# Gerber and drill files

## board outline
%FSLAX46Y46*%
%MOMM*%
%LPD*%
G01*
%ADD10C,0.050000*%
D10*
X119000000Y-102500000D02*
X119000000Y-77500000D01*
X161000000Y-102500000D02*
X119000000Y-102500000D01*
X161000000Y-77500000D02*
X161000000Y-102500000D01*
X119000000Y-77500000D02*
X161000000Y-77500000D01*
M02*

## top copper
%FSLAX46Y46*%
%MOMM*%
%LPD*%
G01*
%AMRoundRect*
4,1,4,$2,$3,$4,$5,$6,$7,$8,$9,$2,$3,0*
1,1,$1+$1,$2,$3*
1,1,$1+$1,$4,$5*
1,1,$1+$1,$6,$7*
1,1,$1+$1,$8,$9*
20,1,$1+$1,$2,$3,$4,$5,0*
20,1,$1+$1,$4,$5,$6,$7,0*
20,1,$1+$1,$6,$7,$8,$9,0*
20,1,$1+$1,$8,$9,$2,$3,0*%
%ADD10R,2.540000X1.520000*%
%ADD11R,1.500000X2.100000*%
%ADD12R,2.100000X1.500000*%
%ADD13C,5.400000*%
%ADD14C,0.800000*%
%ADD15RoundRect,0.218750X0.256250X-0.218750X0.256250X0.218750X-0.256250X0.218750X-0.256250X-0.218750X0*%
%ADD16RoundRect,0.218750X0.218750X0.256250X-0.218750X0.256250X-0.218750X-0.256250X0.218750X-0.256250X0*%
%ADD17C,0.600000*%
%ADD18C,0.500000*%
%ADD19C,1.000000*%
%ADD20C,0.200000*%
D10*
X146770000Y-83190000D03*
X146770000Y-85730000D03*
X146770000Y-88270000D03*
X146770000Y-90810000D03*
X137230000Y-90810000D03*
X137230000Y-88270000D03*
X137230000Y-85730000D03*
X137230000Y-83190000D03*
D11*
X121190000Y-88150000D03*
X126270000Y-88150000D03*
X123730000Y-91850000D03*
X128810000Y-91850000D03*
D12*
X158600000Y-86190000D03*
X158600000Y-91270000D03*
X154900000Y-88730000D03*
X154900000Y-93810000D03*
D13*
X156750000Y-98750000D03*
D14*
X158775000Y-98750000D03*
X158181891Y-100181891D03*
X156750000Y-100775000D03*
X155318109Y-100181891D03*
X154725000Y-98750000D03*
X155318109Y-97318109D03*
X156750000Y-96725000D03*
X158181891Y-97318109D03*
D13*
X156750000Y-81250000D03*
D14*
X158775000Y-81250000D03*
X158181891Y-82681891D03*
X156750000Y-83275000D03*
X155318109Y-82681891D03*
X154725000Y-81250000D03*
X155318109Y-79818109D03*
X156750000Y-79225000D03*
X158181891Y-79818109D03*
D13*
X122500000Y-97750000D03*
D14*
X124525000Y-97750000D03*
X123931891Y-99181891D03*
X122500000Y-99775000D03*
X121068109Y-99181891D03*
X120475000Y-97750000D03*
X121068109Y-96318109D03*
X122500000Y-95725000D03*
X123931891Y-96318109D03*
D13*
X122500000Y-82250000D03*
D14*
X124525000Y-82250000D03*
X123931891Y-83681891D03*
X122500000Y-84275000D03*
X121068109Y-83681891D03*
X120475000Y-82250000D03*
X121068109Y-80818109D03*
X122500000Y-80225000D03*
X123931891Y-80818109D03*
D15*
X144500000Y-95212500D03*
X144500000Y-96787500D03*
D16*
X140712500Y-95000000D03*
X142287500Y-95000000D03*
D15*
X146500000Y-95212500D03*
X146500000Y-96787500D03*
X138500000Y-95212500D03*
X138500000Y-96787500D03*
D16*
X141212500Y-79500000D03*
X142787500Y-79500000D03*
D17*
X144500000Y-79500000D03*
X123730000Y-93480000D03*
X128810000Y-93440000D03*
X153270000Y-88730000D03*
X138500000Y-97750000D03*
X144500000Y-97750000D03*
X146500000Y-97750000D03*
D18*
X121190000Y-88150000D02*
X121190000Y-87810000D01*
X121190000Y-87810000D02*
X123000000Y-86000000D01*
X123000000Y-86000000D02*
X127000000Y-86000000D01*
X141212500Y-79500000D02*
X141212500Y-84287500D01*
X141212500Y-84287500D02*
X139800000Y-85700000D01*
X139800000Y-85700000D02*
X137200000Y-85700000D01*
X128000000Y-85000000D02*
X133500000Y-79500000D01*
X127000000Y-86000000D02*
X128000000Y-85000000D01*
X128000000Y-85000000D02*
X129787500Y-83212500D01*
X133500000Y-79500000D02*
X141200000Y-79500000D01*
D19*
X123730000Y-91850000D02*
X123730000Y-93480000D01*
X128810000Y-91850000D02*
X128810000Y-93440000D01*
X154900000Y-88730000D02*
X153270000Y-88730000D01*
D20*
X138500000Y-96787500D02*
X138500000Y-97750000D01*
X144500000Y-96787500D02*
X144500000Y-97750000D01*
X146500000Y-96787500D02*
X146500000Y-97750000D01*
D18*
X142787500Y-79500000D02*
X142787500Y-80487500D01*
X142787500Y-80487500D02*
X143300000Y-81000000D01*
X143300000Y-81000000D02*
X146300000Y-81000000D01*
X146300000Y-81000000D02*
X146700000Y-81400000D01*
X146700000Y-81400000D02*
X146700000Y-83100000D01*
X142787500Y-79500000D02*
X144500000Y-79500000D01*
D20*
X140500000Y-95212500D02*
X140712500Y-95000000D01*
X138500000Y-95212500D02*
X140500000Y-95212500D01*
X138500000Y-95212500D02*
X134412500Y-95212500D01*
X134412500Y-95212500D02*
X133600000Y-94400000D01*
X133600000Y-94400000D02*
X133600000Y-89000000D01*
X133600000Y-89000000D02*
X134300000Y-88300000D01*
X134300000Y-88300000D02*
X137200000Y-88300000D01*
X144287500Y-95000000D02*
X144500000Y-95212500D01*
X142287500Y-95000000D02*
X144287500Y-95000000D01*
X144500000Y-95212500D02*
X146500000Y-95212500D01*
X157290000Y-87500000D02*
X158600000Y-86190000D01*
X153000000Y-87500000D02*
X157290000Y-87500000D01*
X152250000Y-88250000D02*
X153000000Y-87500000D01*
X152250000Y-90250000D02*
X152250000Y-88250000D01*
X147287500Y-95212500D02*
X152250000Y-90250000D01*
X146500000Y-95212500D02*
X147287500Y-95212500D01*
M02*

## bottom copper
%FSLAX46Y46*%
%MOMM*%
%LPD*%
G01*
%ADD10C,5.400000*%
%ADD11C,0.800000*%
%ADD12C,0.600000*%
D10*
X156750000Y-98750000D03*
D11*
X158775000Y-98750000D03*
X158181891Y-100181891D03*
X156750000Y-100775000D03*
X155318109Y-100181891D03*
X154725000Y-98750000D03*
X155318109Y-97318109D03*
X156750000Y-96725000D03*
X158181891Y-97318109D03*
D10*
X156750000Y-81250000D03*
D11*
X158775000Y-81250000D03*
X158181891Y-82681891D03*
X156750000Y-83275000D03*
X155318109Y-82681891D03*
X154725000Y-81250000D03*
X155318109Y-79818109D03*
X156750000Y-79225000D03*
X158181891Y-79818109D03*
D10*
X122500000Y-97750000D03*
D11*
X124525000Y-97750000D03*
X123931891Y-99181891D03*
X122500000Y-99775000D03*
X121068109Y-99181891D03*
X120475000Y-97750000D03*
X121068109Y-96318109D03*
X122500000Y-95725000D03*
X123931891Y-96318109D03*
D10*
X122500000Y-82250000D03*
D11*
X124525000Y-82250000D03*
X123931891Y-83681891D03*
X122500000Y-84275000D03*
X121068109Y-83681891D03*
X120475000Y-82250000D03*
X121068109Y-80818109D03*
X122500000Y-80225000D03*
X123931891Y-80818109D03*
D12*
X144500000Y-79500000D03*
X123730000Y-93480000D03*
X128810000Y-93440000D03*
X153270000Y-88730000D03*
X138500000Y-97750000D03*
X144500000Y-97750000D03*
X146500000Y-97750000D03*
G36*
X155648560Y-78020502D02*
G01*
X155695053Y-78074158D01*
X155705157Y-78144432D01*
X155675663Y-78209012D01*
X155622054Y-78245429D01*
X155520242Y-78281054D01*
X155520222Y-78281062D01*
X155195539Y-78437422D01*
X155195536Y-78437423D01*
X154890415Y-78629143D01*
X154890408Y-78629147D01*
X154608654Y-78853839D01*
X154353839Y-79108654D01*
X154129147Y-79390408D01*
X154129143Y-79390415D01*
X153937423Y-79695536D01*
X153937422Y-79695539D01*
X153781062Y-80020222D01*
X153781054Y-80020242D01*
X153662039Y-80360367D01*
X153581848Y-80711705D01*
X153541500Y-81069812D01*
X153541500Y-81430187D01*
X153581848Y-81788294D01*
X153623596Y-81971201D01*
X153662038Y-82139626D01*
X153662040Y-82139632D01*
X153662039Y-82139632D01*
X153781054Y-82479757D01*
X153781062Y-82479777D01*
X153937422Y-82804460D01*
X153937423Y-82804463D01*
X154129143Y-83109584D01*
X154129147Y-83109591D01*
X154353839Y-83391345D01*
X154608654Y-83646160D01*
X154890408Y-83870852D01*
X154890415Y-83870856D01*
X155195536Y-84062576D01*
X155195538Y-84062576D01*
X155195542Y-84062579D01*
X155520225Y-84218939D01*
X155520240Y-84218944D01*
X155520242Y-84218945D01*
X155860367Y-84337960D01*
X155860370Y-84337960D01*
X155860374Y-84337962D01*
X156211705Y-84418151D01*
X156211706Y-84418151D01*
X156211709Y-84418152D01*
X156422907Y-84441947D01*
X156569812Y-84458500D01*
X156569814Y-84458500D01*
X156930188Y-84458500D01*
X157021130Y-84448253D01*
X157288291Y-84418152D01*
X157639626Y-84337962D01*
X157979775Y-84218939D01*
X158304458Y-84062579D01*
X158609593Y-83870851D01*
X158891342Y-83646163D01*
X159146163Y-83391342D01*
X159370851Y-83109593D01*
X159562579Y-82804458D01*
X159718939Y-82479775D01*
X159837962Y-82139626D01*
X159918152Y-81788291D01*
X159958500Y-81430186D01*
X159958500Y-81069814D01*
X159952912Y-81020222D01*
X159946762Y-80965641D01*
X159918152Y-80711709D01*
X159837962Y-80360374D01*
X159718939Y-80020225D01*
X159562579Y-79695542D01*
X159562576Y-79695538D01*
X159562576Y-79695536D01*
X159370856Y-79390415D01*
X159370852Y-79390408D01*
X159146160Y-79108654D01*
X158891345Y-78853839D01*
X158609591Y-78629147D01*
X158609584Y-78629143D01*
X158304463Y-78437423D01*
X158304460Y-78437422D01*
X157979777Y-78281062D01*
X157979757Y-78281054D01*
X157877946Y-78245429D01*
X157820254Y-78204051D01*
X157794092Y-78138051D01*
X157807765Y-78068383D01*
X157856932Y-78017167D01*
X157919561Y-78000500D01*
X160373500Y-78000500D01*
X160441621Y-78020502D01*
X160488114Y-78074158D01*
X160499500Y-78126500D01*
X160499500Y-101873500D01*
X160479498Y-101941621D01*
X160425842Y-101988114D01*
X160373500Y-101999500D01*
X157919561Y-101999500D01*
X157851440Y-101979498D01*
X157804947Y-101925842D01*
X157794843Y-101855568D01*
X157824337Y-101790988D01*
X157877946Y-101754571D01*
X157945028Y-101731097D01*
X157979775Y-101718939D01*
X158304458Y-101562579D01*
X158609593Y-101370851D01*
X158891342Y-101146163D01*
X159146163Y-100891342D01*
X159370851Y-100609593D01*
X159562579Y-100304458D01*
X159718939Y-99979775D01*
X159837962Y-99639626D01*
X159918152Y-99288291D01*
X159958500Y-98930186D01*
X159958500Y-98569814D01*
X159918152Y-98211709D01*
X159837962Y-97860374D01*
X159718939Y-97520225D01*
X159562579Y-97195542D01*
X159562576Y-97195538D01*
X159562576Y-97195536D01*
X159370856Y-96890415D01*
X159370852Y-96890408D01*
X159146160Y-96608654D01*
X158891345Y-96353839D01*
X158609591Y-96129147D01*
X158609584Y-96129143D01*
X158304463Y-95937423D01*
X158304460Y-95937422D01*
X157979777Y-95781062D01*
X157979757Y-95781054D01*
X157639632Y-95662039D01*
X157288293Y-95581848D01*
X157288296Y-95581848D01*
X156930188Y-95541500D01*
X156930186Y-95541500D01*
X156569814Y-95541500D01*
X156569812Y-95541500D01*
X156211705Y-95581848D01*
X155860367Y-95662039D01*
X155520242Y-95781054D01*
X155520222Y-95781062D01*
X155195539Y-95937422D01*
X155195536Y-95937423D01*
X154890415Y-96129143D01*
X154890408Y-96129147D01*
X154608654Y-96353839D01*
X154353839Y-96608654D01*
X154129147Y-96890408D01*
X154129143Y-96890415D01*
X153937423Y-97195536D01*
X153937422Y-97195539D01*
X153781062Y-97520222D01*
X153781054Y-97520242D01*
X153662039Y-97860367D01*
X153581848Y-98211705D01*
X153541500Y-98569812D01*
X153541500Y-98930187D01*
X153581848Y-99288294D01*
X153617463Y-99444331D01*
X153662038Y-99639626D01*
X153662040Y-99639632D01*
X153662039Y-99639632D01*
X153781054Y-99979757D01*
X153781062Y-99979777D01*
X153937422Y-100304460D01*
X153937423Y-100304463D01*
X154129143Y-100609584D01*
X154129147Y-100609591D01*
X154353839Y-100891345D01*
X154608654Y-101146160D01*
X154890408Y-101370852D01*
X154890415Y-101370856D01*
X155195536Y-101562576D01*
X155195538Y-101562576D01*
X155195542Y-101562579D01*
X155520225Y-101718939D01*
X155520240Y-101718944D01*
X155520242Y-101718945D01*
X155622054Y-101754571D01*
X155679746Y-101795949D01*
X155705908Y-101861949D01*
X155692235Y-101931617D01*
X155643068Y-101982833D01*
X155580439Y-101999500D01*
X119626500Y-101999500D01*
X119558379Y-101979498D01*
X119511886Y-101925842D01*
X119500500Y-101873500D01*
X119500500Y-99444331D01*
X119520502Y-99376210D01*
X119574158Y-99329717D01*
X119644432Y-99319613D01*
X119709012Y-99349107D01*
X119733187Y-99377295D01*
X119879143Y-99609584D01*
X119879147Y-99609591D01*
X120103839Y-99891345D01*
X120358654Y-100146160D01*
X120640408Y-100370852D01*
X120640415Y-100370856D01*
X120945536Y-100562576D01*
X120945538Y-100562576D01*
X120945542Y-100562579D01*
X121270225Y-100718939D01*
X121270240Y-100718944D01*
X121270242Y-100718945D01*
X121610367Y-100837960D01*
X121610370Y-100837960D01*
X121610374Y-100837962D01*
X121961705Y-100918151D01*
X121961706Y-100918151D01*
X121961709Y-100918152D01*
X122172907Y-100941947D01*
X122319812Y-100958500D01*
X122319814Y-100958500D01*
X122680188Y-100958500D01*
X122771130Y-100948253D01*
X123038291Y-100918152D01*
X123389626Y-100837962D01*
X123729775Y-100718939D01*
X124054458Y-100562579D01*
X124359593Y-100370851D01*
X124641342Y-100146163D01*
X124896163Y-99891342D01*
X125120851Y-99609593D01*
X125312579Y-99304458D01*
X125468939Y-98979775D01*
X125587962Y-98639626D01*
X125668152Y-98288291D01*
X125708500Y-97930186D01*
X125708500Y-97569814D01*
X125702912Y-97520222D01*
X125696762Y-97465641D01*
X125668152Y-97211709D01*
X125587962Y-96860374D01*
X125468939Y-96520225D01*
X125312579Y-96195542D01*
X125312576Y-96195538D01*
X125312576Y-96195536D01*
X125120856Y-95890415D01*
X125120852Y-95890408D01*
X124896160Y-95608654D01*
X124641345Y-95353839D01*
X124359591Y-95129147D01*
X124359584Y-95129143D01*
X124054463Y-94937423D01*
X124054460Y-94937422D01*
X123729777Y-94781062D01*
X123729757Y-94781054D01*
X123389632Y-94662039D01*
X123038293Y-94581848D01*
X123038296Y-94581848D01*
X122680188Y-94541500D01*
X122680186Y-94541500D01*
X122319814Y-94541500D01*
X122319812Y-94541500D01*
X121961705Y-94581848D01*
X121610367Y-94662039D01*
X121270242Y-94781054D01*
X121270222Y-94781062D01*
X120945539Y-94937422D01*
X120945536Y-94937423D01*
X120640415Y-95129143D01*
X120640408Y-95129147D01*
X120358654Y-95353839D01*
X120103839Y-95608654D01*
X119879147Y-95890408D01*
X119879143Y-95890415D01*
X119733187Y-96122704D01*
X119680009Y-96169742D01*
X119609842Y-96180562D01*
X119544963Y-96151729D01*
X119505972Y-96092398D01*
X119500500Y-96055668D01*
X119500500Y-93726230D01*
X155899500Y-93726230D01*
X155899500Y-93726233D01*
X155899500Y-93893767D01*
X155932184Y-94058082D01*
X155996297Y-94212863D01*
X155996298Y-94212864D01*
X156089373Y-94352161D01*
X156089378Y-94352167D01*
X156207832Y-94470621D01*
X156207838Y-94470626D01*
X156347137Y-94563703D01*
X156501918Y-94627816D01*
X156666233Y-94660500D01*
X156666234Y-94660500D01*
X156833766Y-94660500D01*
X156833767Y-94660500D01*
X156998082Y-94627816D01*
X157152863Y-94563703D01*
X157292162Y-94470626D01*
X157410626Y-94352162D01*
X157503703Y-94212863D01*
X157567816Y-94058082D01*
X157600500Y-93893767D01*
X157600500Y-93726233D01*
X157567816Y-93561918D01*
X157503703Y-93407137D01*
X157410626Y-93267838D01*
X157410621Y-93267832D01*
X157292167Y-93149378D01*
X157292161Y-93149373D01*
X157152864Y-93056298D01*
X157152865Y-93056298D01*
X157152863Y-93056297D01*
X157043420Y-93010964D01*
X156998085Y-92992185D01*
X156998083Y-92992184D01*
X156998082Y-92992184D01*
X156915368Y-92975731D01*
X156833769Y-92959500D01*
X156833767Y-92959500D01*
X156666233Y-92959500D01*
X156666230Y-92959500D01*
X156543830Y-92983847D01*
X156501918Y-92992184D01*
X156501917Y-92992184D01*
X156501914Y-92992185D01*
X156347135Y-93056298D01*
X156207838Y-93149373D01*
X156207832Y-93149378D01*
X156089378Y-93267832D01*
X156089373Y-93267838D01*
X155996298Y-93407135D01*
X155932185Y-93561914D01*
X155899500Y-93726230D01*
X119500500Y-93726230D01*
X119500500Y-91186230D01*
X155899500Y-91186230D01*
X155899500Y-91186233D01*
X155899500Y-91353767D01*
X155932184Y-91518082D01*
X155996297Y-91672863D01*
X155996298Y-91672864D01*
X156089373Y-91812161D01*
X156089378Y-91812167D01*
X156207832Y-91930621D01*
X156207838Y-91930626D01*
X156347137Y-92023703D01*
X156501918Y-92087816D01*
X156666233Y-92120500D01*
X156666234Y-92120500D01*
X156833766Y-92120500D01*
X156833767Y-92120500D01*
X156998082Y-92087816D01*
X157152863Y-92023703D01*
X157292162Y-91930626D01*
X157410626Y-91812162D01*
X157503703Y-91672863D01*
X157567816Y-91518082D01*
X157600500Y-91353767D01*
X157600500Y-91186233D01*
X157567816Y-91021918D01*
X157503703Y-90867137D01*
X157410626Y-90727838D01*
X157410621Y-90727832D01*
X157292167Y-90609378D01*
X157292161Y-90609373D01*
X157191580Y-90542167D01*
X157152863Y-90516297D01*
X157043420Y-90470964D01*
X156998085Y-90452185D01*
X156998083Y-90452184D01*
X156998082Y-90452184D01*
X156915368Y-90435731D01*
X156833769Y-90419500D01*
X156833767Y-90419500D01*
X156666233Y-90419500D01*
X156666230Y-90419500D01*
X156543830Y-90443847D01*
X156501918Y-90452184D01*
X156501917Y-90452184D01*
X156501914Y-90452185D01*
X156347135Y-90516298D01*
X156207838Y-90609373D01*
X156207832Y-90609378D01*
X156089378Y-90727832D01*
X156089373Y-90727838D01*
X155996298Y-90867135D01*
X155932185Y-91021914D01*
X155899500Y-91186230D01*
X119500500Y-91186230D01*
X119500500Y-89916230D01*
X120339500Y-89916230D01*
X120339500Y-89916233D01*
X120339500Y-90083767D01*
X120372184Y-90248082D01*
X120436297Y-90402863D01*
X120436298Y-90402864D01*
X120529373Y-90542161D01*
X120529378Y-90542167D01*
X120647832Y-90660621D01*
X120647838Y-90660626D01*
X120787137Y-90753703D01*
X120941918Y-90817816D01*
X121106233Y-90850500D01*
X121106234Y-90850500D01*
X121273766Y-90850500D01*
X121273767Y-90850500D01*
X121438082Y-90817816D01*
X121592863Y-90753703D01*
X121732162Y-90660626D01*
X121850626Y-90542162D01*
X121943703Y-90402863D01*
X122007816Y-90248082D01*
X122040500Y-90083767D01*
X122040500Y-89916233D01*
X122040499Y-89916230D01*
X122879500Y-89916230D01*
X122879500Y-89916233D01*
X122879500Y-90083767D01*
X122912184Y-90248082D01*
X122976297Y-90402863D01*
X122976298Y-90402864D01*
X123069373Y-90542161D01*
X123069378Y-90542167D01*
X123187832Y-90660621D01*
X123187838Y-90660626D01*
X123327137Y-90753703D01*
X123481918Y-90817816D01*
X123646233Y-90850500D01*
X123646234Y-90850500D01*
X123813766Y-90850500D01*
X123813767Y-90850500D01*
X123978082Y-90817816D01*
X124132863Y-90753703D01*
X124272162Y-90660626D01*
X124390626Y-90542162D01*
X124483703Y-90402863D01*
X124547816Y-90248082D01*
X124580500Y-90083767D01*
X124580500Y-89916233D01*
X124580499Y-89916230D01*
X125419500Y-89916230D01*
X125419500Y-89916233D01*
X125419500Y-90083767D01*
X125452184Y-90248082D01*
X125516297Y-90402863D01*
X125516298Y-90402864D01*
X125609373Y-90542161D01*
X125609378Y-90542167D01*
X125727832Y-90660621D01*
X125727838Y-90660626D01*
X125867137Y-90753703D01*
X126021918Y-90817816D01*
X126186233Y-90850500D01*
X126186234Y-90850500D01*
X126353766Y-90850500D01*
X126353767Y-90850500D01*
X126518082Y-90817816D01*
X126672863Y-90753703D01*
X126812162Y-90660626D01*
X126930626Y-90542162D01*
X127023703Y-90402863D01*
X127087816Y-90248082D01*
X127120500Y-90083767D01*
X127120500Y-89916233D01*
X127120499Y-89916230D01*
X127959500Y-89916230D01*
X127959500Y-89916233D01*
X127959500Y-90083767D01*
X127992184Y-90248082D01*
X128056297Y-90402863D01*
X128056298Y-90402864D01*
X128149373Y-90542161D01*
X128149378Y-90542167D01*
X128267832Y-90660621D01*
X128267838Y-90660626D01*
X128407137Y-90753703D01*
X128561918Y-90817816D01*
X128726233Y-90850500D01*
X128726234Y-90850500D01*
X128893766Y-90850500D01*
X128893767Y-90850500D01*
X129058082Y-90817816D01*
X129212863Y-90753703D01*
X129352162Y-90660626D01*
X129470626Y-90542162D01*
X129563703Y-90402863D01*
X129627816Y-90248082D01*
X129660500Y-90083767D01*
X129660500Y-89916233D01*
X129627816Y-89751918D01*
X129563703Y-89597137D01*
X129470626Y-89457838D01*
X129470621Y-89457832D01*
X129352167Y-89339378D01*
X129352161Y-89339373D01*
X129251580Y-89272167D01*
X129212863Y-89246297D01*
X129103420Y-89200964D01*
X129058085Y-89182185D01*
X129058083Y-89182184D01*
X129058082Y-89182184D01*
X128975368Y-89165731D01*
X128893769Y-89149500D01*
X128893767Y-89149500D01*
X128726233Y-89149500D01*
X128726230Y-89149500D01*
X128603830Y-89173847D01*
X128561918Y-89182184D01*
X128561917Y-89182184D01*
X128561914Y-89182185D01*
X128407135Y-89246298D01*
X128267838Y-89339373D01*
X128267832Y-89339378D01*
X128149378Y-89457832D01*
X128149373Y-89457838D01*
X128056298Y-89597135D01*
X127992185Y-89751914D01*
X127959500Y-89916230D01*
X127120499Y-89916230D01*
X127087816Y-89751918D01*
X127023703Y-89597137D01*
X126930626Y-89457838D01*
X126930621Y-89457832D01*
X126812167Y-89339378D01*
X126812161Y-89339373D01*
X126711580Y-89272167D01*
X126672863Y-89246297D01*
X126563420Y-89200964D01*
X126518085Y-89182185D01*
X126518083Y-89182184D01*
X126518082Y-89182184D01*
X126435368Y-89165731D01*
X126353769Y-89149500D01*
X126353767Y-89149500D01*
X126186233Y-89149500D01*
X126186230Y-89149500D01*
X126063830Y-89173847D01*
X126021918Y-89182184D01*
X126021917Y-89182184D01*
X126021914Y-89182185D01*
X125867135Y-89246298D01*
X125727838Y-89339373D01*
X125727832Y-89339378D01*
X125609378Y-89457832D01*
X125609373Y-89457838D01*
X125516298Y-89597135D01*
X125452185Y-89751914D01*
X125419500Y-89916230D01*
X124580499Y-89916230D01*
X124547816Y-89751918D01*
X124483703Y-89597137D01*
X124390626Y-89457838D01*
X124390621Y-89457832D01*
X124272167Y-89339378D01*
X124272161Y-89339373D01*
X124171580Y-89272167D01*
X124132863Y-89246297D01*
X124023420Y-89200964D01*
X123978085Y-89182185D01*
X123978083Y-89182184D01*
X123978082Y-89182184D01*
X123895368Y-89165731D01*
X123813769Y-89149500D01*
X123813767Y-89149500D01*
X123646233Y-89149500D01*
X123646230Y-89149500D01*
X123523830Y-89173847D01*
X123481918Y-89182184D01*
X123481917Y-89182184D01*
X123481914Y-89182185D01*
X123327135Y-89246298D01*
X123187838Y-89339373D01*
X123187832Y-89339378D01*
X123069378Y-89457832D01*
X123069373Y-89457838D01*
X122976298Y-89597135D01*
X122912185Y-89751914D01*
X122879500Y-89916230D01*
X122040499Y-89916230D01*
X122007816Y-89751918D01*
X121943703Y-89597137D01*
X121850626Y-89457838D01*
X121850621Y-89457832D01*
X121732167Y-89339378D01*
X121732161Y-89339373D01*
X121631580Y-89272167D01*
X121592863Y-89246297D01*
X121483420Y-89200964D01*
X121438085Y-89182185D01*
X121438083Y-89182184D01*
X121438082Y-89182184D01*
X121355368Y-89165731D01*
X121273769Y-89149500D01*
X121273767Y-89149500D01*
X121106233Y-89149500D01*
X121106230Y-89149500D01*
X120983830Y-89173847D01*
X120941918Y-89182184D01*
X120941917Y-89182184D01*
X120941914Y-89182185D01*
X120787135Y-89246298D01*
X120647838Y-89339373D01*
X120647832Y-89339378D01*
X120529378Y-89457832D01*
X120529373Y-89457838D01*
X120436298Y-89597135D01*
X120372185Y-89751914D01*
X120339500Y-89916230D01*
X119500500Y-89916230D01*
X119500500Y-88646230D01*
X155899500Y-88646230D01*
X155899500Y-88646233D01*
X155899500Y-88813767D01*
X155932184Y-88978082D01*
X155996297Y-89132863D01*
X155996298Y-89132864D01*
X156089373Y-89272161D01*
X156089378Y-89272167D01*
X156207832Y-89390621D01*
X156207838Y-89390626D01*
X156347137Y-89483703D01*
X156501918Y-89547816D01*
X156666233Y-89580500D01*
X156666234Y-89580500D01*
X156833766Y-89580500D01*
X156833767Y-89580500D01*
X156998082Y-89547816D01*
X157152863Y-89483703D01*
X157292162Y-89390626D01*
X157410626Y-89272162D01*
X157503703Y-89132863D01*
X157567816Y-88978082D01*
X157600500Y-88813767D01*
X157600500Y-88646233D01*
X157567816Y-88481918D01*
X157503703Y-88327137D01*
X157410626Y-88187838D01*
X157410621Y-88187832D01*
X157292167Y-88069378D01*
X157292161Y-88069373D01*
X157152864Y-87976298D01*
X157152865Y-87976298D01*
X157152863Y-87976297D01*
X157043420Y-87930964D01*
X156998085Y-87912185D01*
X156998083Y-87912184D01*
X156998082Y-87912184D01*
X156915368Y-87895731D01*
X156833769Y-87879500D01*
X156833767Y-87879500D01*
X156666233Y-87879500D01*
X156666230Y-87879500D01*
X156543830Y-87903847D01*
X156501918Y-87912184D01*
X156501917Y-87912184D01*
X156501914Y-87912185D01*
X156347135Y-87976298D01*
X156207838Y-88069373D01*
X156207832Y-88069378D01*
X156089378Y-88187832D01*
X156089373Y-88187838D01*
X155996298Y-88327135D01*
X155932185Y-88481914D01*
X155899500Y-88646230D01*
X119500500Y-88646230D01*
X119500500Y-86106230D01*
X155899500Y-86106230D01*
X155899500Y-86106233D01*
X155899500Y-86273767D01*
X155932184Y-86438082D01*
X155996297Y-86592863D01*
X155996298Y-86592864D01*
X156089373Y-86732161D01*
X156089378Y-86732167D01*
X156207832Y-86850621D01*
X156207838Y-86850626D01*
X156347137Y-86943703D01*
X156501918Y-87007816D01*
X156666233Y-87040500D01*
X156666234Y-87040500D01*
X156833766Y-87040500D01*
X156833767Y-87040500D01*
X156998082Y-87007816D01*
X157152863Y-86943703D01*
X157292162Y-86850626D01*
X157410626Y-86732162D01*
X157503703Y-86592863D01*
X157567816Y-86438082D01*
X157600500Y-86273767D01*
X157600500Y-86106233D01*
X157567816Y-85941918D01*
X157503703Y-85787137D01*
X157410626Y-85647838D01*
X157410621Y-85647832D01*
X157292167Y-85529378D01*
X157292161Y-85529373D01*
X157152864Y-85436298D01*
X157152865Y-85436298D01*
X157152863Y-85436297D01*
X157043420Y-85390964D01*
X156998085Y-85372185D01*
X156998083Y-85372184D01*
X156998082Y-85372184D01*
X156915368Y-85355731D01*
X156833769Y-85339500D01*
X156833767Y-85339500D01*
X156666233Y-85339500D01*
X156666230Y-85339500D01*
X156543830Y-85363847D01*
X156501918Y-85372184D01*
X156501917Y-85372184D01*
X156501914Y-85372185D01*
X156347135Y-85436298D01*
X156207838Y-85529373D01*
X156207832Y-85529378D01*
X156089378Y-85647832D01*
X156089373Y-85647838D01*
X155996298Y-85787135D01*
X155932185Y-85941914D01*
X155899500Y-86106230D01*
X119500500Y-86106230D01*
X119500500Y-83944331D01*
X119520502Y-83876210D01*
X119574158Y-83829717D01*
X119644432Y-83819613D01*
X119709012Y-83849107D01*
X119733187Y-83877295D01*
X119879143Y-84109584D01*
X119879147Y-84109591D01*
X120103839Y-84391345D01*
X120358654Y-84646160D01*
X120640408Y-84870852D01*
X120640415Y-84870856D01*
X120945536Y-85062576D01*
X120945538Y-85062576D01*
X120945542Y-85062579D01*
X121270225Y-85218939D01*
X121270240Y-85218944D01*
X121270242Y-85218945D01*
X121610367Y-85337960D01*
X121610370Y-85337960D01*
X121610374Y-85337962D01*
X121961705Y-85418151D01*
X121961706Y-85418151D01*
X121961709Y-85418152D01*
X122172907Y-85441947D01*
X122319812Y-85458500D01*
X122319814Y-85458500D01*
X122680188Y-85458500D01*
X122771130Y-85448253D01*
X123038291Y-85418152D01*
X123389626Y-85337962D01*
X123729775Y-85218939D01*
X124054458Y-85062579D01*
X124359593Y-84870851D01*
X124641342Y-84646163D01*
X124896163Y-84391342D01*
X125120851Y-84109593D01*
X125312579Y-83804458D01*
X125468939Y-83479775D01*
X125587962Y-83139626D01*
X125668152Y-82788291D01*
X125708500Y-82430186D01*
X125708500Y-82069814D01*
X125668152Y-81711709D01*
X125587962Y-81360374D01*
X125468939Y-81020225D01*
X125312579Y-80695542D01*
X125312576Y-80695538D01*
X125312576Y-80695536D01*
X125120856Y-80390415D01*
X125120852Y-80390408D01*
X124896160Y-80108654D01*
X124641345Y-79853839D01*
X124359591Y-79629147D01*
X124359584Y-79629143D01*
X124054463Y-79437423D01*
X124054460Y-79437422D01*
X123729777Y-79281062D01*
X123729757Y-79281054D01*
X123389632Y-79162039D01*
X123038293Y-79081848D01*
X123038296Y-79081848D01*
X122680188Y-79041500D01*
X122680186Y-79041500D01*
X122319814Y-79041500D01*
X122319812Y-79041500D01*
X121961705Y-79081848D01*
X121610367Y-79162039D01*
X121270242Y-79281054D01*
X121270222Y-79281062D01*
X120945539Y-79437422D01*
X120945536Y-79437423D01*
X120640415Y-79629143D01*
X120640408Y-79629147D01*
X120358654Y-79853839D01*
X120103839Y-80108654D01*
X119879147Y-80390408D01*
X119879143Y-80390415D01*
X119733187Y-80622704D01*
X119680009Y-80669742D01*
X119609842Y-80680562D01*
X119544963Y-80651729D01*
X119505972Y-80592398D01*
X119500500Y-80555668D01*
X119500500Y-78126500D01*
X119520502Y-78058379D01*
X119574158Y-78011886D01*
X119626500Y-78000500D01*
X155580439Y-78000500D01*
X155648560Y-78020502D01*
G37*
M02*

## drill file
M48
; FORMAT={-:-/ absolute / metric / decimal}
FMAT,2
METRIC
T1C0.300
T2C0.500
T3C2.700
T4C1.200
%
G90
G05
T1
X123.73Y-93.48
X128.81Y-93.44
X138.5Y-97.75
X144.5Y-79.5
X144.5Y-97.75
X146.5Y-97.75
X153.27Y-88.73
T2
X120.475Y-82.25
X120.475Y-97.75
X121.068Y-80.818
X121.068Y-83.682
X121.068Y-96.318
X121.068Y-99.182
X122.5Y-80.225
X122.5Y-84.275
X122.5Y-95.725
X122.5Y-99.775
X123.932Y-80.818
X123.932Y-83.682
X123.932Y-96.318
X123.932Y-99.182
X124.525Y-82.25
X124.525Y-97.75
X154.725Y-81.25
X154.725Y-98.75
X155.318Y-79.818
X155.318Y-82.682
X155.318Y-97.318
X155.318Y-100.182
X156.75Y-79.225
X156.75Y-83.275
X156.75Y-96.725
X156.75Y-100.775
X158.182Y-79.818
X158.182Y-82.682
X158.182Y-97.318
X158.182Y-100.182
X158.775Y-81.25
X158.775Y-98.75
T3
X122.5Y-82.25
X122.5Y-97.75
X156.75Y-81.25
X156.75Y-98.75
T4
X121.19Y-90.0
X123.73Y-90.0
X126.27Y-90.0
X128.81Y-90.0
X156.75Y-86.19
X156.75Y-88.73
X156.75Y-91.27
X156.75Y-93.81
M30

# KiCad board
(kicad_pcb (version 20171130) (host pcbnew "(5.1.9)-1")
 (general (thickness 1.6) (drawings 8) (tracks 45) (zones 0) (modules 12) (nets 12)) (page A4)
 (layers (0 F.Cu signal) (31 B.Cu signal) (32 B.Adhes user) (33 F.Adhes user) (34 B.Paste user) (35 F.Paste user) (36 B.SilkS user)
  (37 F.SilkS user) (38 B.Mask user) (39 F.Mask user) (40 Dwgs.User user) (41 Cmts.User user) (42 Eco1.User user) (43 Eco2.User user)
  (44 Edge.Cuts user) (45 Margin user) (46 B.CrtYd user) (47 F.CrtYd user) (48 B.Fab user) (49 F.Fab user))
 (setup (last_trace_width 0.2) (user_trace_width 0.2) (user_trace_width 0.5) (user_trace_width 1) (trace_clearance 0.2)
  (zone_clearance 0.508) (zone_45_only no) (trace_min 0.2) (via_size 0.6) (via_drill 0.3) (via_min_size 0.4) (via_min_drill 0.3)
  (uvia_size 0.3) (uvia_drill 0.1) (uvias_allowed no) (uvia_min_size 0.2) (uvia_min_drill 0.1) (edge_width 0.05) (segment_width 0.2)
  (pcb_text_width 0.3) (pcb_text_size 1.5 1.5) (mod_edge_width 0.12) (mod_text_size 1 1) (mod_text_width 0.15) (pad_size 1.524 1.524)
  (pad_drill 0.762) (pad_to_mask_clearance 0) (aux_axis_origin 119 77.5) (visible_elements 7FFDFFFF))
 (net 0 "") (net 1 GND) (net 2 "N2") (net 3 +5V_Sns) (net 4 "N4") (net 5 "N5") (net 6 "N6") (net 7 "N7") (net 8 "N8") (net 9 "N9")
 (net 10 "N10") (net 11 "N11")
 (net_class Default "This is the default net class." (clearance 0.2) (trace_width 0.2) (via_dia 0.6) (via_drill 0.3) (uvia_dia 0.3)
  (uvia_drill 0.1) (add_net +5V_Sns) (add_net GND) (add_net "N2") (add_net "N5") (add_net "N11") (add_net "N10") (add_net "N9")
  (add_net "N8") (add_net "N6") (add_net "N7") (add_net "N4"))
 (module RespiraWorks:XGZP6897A (layer F.Cu) (at 142 87)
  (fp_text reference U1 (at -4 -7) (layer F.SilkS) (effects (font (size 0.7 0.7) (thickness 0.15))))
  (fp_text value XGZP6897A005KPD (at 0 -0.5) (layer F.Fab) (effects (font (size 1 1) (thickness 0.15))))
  (pad 8 smd rect (at 4.77 -3.81) (size 2.54 1.52) (layers F.Cu F.Paste F.Mask) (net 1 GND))
  (pad 7 smd rect (at 4.77 -1.27) (size 2.54 1.52) (layers F.Cu F.Paste F.Mask))
  (pad 6 smd rect (at 4.77 1.27) (size 2.54 1.52) (layers F.Cu F.Paste F.Mask))
  (pad 5 smd rect (at 4.77 3.81) (size 2.54 1.52) (layers F.Cu F.Paste F.Mask))
  (pad 4 smd rect (at -4.77 3.81) (size 2.54 1.52) (layers F.Cu F.Paste F.Mask))
  (pad 3 smd rect (at -4.77 1.27) (size 2.54 1.52) (layers F.Cu F.Paste F.Mask) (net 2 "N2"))
  (pad 2 smd rect (at -4.77 -1.27) (size 2.54 1.52) (layers F.Cu F.Paste F.Mask) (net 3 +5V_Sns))
  (pad 1 smd rect (at -4.77 -3.81) (size 2.54 1.52) (layers F.Cu F.Paste F.Mask)))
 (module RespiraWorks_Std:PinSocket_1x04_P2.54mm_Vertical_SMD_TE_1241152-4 (layer F.Cu) (at 125 90 90)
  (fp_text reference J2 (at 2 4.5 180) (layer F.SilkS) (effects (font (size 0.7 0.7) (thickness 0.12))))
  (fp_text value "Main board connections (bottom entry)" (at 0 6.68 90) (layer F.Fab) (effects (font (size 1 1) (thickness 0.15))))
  (pad "" np_thru_hole circle (at 0 1.27 90) (size 1.2 1.2) (drill 1.2) (layers *.Cu *.Mask))
  (pad "" np_thru_hole circle (at 0 -1.27 90) (size 1.2 1.2) (drill 1.2) (layers *.Cu *.Mask))
  (pad "" np_thru_hole circle (at 0 -3.81 90) (size 1.2 1.2) (drill 1.2) (layers *.Cu *.Mask))
  (pad 1 smd rect (at 1.85 -3.81 90) (size 2.1 1.5) (layers F.Cu F.Paste F.Mask) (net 3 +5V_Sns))
  (pad 3 smd rect (at 1.85 1.27 90) (size 2.1 1.5) (layers F.Cu F.Paste F.Mask) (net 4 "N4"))
  (pad 2 smd rect (at -1.85 -1.27 90) (size 2.1 1.5) (layers F.Cu F.Paste F.Mask) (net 1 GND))
  (pad 4 smd rect (at -1.85 3.81 90) (size 2.1 1.5) (layers F.Cu F.Paste F.Mask) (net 1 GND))
  (pad "" np_thru_hole circle (at 0 3.81 90) (size 1.2 1.2) (drill 1.2) (layers *.Cu *.Mask)))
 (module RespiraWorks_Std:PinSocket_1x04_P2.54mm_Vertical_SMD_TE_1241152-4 (layer F.Cu) (at 156.75 90)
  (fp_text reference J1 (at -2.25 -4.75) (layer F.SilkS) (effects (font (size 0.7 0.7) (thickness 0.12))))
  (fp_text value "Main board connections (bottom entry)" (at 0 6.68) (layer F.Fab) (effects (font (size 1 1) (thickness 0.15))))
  (pad "" np_thru_hole circle (at 0 1.27) (size 1.2 1.2) (drill 1.2) (layers *.Cu *.Mask))
  (pad "" np_thru_hole circle (at 0 -1.27) (size 1.2 1.2) (drill 1.2) (layers *.Cu *.Mask))
  (pad "" np_thru_hole circle (at 0 -3.81) (size 1.2 1.2) (drill 1.2) (layers *.Cu *.Mask))
  (pad 1 smd rect (at 1.85 -3.81) (size 2.1 1.5) (layers F.Cu F.Paste F.Mask) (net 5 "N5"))
  (pad 3 smd rect (at 1.85 1.27) (size 2.1 1.5) (layers F.Cu F.Paste F.Mask) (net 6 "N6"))
  (pad 2 smd rect (at -1.85 -1.27) (size 2.1 1.5) (layers F.Cu F.Paste F.Mask) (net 1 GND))
  (pad 4 smd rect (at -1.85 3.81) (size 2.1 1.5) (layers F.Cu F.Paste F.Mask) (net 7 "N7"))
  (pad "" np_thru_hole circle (at 0 3.81) (size 1.2 1.2) (drill 1.2) (layers *.Cu *.Mask)))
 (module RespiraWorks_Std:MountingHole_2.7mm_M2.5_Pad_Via (layer F.Cu) (at 156.75 98.75)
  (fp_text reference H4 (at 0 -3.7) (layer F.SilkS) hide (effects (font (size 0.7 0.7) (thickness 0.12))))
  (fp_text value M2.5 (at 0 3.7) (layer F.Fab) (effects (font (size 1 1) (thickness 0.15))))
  (pad 1 thru_hole circle (at 0 0) (size 5.4 5.4) (drill 2.7) (layers *.Cu *.Mask) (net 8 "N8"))
  (pad 1 thru_hole circle (at 2.025 0) (size 0.8 0.8) (drill 0.5) (layers *.Cu *.Mask) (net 8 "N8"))
  (pad 1 thru_hole circle (at 1.431891 1.431891) (size 0.8 0.8) (drill 0.5) (layers *.Cu *.Mask) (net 8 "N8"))
  (pad 1 thru_hole circle (at 0 2.025) (size 0.8 0.8) (drill 0.5) (layers *.Cu *.Mask) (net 8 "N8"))
  (pad 1 thru_hole circle (at -1.431891 1.431891) (size 0.8 0.8) (drill 0.5) (layers *.Cu *.Mask) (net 8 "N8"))
  (pad 1 thru_hole circle (at -2.025 0) (size 0.8 0.8) (drill 0.5) (layers *.Cu *.Mask) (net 8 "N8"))
  (pad 1 thru_hole circle (at -1.431891 -1.431891) (size 0.8 0.8) (drill 0.5) (layers *.Cu *.Mask) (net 8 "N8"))
  (pad 1 thru_hole circle (at 0 -2.025) (size 0.8 0.8) (drill 0.5) (layers *.Cu *.Mask) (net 8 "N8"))
  (pad 1 thru_hole circle (at 1.431891 -1.431891) (size 0.8 0.8) (drill 0.5) (layers *.Cu *.Mask) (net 8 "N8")))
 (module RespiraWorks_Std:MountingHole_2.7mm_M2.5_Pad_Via (layer F.Cu) (at 156.75 81.25)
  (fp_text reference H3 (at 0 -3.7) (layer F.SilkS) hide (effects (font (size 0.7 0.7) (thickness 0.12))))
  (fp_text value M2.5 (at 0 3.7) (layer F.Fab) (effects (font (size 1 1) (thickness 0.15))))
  (pad 1 thru_hole circle (at 0 0) (size 5.4 5.4) (drill 2.7) (layers *.Cu *.Mask) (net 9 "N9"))
  (pad 1 thru_hole circle (at 2.025 0) (size 0.8 0.8) (drill 0.5) (layers *.Cu *.Mask) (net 9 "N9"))
  (pad 1 thru_hole circle (at 1.431891 1.431891) (size 0.8 0.8) (drill 0.5) (layers *.Cu *.Mask) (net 9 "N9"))
  (pad 1 thru_hole circle (at 0 2.025) (size 0.8 0.8) (drill 0.5) (layers *.Cu *.Mask) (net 9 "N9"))
  (pad 1 thru_hole circle (at -1.431891 1.431891) (size 0.8 0.8) (drill 0.5) (layers *.Cu *.Mask) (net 9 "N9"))
  (pad 1 thru_hole circle (at -2.025 0) (size 0.8 0.8) (drill 0.5) (layers *.Cu *.Mask) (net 9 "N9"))
  (pad 1 thru_hole circle (at -1.431891 -1.431891) (size 0.8 0.8) (drill 0.5) (layers *.Cu *.Mask) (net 9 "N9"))
  (pad 1 thru_hole circle (at 0 -2.025) (size 0.8 0.8) (drill 0.5) (layers *.Cu *.Mask) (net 9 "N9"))
  (pad 1 thru_hole circle (at 1.431891 -1.431891) (size 0.8 0.8) (drill 0.5) (layers *.Cu *.Mask) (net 9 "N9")))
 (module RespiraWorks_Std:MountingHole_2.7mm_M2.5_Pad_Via (layer F.Cu) (at 122.5 97.75)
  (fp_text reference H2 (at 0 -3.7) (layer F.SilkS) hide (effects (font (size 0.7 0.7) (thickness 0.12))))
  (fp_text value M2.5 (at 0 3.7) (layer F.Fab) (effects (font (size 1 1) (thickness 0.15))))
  (pad 1 thru_hole circle (at 0 0) (size 5.4 5.4) (drill 2.7) (layers *.Cu *.Mask) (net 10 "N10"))
  (pad 1 thru_hole circle (at 2.025 0) (size 0.8 0.8) (drill 0.5) (layers *.Cu *.Mask) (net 10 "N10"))
  (pad 1 thru_hole circle (at 1.431891 1.431891) (size 0.8 0.8) (drill 0.5) (layers *.Cu *.Mask) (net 10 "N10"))
  (pad 1 thru_hole circle (at 0 2.025) (size 0.8 0.8) (drill 0.5) (layers *.Cu *.Mask) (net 10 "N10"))
  (pad 1 thru_hole circle (at -1.431891 1.431891) (size 0.8 0.8) (drill 0.5) (layers *.Cu *.Mask) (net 10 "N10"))
  (pad 1 thru_hole circle (at -2.025 0) (size 0.8 0.8) (drill 0.5) (layers *.Cu *.Mask) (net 10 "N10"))
  (pad 1 thru_hole circle (at -1.431891 -1.431891) (size 0.8 0.8) (drill 0.5) (layers *.Cu *.Mask) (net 10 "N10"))
  (pad 1 thru_hole circle (at 0 -2.025) (size 0.8 0.8) (drill 0.5) (layers *.Cu *.Mask) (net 10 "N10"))
  (pad 1 thru_hole circle (at 1.431891 -1.431891) (size 0.8 0.8) (drill 0.5) (layers *.Cu *.Mask) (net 10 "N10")))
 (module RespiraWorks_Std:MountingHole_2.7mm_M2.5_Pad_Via (layer F.Cu) (at 122.5 82.25)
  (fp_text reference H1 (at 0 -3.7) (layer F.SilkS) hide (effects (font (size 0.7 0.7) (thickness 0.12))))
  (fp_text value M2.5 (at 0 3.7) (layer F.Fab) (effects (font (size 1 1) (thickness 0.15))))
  (pad 1 thru_hole circle (at 0 0) (size 5.4 5.4) (drill 2.7) (layers *.Cu *.Mask) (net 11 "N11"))
  (pad 1 thru_hole circle (at 2.025 0) (size 0.8 0.8) (drill 0.5) (layers *.Cu *.Mask) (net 11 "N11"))
  (pad 1 thru_hole circle (at 1.431891 1.431891) (size 0.8 0.8) (drill 0.5) (layers *.Cu *.Mask) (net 11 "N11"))
  (pad 1 thru_hole circle (at 0 2.025) (size 0.8 0.8) (drill 0.5) (layers *.Cu *.Mask) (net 11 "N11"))
  (pad 1 thru_hole circle (at -1.431891 1.431891) (size 0.8 0.8) (drill 0.5) (layers *.Cu *.Mask) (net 11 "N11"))
  (pad 1 thru_hole circle (at -2.025 0) (size 0.8 0.8) (drill 0.5) (layers *.Cu *.Mask) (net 11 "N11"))
  (pad 1 thru_hole circle (at -1.431891 -1.431891) (size 0.8 0.8) (drill 0.5) (layers *.Cu *.Mask) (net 11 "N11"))
  (pad 1 thru_hole circle (at 0 -2.025) (size 0.8 0.8) (drill 0.5) (layers *.Cu *.Mask) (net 11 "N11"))
  (pad 1 thru_hole circle (at 1.431891 -1.431891) (size 0.8 0.8) (drill 0.5) (layers *.Cu *.Mask) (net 11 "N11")))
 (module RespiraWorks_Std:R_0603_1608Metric (layer F.Cu) (at 144.5 96 90)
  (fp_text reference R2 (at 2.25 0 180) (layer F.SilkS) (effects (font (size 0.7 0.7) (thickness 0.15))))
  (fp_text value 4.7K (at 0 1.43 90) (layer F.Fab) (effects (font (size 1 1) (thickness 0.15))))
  (pad 2 smd roundrect (at 0.7875 0 90) (size 0.875 0.95) (layers F.Cu F.Paste F.Mask) (roundrect_rratio 0.25) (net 5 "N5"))
  (pad 1 smd roundrect (at -0.7875 0 90) (size 0.875 0.95) (layers F.Cu F.Paste F.Mask) (roundrect_rratio 0.25) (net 1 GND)))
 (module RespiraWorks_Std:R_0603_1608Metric (layer F.Cu) (at 141.5 95 180)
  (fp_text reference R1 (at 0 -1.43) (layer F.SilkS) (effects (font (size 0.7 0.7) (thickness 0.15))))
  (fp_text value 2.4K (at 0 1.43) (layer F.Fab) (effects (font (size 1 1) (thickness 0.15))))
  (pad 2 smd roundrect (at 0.7875 0 180) (size 0.875 0.95) (layers F.Cu F.Paste F.Mask) (roundrect_rratio 0.25) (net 2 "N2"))
  (pad 1 smd roundrect (at -0.7875 0 180) (size 0.875 0.95) (layers F.Cu F.Paste F.Mask) (roundrect_rratio 0.25) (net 5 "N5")))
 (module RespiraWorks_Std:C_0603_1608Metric (layer F.Cu) (at 146.5 96 90)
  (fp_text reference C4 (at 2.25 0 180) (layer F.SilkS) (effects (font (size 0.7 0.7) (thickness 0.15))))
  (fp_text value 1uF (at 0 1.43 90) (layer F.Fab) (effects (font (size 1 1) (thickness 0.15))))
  (pad 2 smd roundrect (at 0.7875 0 90) (size 0.875 0.95) (layers F.Cu F.Paste F.Mask) (roundrect_rratio 0.25) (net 5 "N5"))
  (pad 1 smd roundrect (at -0.7875 0 90) (size 0.875 0.95) (layers F.Cu F.Paste F.Mask) (roundrect_rratio 0.25) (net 1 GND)))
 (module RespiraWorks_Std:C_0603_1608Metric (layer F.Cu) (at 138.5 96 90)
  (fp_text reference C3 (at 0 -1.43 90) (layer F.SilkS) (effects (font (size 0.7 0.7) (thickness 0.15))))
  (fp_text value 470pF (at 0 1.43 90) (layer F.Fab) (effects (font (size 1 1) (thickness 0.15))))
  (pad 2 smd roundrect (at 0.7875 0 90) (size 0.875 0.95) (layers F.Cu F.Paste F.Mask) (roundrect_rratio 0.25) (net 2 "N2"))
  (pad 1 smd roundrect (at -0.7875 0 90) (size 0.875 0.95) (layers F.Cu F.Paste F.Mask) (roundrect_rratio 0.25) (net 1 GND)))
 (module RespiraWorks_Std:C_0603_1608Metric (layer F.Cu) (at 142 79.5 180)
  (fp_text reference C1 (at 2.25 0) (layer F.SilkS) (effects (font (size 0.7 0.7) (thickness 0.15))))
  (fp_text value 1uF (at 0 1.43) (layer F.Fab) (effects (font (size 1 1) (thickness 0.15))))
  (pad 2 smd roundrect (at 0.7875 0 180) (size 0.875 0.95) (layers F.Cu F.Paste F.Mask) (roundrect_rratio 0.25) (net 3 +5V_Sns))
  (pad 1 smd roundrect (at -0.7875 0 180) (size 0.875 0.95) (layers F.Cu F.Paste F.Mask) (roundrect_rratio 0.25) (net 1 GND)))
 (gr_line (start 119 102.5) (end 119 77.5) (layer Edge.Cuts) (width 0.05))
 (gr_line (start 161 102.5) (end 119 102.5) (layer Edge.Cuts) (width 0.05))
 (gr_line (start 161 77.5) (end 161 102.5) (layer Edge.Cuts) (width 0.05))
 (gr_line (start 119 77.5) (end 161 77.5) (layer Edge.Cuts) (width 0.05))
 (segment (start 121.19 88.15) (end 121.19 87.81) (width 0.5) (layer F.Cu) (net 3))
 (segment (start 121.19 87.81) (end 123 86) (width 0.5) (layer F.Cu) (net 3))
 (segment (start 123 86) (end 127 86) (width 0.5) (layer F.Cu) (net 3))
 (segment (start 141.2125 79.5) (end 141.2125 84.2875) (width 0.5) (layer F.Cu) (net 3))
 (segment (start 141.2125 84.2875) (end 139.8 85.7) (width 0.5) (layer F.Cu) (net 3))
 (segment (start 139.8 85.7) (end 137.2 85.7) (width 0.5) (layer F.Cu) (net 3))
 (segment (start 128 85) (end 133.5 79.5) (width 0.5) (layer F.Cu) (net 3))
 (segment (start 127 86) (end 128 85) (width 0.5) (layer F.Cu) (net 3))
 (segment (start 128 85) (end 129.7875 83.2125) (width 0.5) (layer F.Cu) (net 3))
 (segment (start 133.5 79.5) (end 141.2 79.5) (width 0.5) (layer F.Cu) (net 3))
 (via (at 144.5 79.5) (size 0.6) (drill 0.3) (layers F.Cu B.Cu) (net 1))
 (segment (start 123.73 91.85) (end 123.73 93.48) (width 1) (layer F.Cu) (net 1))
 (via (at 123.73 93.48) (size 0.6) (drill 0.3) (layers F.Cu B.Cu) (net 1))
 (segment (start 128.81 91.85) (end 128.81 93.44) (width 1) (layer F.Cu) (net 1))
 (via (at 128.81 93.44) (size 0.6) (drill 0.3) (layers F.Cu B.Cu) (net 1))
 (segment (start 154.9 88.73) (end 153.27 88.73) (width 1) (layer F.Cu) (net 1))
 (via (at 153.27 88.73) (size 0.6) (drill 0.3) (layers F.Cu B.Cu) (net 1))
 (segment (start 138.5 96.7875) (end 138.5 97.75) (width 0.2) (layer F.Cu) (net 1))
 (via (at 138.5 97.75) (size 0.6) (drill 0.3) (layers F.Cu B.Cu) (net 1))
 (segment (start 144.5 96.7875) (end 144.5 97.75) (width 0.2) (layer F.Cu) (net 1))
 (via (at 144.5 97.75) (size 0.6) (drill 0.3) (layers F.Cu B.Cu) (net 1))
 (segment (start 146.5 96.7875) (end 146.5 97.75) (width 0.2) (layer F.Cu) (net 1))
 (via (at 146.5 97.75) (size 0.6) (drill 0.3) (layers F.Cu B.Cu) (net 1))
 (segment (start 142.7875 79.5) (end 142.7875 80.4875) (width 0.5) (layer F.Cu) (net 1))
 (segment (start 142.7875 80.4875) (end 143.3 81) (width 0.5) (layer F.Cu) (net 1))
 (segment (start 143.3 81) (end 146.3 81) (width 0.5) (layer F.Cu) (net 1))
 (segment (start 146.3 81) (end 146.7 81.4) (width 0.5) (layer F.Cu) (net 1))
 (segment (start 146.7 81.4) (end 146.7 83.1) (width 0.5) (layer F.Cu) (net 1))
 (segment (start 142.7875 79.5) (end 144.5 79.5) (width 0.5) (layer F.Cu) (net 1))
 (segment (start 140.5 95.2125) (end 140.7125 95) (width 0.2) (layer F.Cu) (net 2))
 (segment (start 138.5 95.2125) (end 140.5 95.2125) (width 0.2) (layer F.Cu) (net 2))
 (segment (start 138.5 95.2125) (end 134.4125 95.2125) (width 0.2) (layer F.Cu) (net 2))
 (segment (start 134.4125 95.2125) (end 133.6 94.4) (width 0.2) (layer F.Cu) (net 2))
 (segment (start 133.6 94.4) (end 133.6 89) (width 0.2) (layer F.Cu) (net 2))
 (segment (start 133.6 89) (end 134.3 88.3) (width 0.2) (layer F.Cu) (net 2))
 (segment (start 134.3 88.3) (end 137.2 88.3) (width 0.2) (layer F.Cu) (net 2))
 (segment (start 144.2875 95) (end 144.5 95.2125) (width 0.2) (layer F.Cu) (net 5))
 (segment (start 142.2875 95) (end 144.2875 95) (width 0.2) (layer F.Cu) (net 5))
 (segment (start 144.5 95.2125) (end 146.5 95.2125) (width 0.2) (layer F.Cu) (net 5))
 (segment (start 157.29 87.5) (end 158.6 86.19) (width 0.2) (layer F.Cu) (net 5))
 (segment (start 153 87.5) (end 157.29 87.5) (width 0.2) (layer F.Cu) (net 5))
 (segment (start 152.25 88.25) (end 153 87.5) (width 0.2) (layer F.Cu) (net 5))
 (segment (start 152.25 90.25) (end 152.25 88.25) (width 0.2) (layer F.Cu) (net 5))
 (segment (start 147.2875 95.2125) (end 152.25 90.25) (width 0.2) (layer F.Cu) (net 5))
 (segment (start 146.5 95.2125) (end 147.2875 95.2125) (width 0.2) (layer F.Cu) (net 5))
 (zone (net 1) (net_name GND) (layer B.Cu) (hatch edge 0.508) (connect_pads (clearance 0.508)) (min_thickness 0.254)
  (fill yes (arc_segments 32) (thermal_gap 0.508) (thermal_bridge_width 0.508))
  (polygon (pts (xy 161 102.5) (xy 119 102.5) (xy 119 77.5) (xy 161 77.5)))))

